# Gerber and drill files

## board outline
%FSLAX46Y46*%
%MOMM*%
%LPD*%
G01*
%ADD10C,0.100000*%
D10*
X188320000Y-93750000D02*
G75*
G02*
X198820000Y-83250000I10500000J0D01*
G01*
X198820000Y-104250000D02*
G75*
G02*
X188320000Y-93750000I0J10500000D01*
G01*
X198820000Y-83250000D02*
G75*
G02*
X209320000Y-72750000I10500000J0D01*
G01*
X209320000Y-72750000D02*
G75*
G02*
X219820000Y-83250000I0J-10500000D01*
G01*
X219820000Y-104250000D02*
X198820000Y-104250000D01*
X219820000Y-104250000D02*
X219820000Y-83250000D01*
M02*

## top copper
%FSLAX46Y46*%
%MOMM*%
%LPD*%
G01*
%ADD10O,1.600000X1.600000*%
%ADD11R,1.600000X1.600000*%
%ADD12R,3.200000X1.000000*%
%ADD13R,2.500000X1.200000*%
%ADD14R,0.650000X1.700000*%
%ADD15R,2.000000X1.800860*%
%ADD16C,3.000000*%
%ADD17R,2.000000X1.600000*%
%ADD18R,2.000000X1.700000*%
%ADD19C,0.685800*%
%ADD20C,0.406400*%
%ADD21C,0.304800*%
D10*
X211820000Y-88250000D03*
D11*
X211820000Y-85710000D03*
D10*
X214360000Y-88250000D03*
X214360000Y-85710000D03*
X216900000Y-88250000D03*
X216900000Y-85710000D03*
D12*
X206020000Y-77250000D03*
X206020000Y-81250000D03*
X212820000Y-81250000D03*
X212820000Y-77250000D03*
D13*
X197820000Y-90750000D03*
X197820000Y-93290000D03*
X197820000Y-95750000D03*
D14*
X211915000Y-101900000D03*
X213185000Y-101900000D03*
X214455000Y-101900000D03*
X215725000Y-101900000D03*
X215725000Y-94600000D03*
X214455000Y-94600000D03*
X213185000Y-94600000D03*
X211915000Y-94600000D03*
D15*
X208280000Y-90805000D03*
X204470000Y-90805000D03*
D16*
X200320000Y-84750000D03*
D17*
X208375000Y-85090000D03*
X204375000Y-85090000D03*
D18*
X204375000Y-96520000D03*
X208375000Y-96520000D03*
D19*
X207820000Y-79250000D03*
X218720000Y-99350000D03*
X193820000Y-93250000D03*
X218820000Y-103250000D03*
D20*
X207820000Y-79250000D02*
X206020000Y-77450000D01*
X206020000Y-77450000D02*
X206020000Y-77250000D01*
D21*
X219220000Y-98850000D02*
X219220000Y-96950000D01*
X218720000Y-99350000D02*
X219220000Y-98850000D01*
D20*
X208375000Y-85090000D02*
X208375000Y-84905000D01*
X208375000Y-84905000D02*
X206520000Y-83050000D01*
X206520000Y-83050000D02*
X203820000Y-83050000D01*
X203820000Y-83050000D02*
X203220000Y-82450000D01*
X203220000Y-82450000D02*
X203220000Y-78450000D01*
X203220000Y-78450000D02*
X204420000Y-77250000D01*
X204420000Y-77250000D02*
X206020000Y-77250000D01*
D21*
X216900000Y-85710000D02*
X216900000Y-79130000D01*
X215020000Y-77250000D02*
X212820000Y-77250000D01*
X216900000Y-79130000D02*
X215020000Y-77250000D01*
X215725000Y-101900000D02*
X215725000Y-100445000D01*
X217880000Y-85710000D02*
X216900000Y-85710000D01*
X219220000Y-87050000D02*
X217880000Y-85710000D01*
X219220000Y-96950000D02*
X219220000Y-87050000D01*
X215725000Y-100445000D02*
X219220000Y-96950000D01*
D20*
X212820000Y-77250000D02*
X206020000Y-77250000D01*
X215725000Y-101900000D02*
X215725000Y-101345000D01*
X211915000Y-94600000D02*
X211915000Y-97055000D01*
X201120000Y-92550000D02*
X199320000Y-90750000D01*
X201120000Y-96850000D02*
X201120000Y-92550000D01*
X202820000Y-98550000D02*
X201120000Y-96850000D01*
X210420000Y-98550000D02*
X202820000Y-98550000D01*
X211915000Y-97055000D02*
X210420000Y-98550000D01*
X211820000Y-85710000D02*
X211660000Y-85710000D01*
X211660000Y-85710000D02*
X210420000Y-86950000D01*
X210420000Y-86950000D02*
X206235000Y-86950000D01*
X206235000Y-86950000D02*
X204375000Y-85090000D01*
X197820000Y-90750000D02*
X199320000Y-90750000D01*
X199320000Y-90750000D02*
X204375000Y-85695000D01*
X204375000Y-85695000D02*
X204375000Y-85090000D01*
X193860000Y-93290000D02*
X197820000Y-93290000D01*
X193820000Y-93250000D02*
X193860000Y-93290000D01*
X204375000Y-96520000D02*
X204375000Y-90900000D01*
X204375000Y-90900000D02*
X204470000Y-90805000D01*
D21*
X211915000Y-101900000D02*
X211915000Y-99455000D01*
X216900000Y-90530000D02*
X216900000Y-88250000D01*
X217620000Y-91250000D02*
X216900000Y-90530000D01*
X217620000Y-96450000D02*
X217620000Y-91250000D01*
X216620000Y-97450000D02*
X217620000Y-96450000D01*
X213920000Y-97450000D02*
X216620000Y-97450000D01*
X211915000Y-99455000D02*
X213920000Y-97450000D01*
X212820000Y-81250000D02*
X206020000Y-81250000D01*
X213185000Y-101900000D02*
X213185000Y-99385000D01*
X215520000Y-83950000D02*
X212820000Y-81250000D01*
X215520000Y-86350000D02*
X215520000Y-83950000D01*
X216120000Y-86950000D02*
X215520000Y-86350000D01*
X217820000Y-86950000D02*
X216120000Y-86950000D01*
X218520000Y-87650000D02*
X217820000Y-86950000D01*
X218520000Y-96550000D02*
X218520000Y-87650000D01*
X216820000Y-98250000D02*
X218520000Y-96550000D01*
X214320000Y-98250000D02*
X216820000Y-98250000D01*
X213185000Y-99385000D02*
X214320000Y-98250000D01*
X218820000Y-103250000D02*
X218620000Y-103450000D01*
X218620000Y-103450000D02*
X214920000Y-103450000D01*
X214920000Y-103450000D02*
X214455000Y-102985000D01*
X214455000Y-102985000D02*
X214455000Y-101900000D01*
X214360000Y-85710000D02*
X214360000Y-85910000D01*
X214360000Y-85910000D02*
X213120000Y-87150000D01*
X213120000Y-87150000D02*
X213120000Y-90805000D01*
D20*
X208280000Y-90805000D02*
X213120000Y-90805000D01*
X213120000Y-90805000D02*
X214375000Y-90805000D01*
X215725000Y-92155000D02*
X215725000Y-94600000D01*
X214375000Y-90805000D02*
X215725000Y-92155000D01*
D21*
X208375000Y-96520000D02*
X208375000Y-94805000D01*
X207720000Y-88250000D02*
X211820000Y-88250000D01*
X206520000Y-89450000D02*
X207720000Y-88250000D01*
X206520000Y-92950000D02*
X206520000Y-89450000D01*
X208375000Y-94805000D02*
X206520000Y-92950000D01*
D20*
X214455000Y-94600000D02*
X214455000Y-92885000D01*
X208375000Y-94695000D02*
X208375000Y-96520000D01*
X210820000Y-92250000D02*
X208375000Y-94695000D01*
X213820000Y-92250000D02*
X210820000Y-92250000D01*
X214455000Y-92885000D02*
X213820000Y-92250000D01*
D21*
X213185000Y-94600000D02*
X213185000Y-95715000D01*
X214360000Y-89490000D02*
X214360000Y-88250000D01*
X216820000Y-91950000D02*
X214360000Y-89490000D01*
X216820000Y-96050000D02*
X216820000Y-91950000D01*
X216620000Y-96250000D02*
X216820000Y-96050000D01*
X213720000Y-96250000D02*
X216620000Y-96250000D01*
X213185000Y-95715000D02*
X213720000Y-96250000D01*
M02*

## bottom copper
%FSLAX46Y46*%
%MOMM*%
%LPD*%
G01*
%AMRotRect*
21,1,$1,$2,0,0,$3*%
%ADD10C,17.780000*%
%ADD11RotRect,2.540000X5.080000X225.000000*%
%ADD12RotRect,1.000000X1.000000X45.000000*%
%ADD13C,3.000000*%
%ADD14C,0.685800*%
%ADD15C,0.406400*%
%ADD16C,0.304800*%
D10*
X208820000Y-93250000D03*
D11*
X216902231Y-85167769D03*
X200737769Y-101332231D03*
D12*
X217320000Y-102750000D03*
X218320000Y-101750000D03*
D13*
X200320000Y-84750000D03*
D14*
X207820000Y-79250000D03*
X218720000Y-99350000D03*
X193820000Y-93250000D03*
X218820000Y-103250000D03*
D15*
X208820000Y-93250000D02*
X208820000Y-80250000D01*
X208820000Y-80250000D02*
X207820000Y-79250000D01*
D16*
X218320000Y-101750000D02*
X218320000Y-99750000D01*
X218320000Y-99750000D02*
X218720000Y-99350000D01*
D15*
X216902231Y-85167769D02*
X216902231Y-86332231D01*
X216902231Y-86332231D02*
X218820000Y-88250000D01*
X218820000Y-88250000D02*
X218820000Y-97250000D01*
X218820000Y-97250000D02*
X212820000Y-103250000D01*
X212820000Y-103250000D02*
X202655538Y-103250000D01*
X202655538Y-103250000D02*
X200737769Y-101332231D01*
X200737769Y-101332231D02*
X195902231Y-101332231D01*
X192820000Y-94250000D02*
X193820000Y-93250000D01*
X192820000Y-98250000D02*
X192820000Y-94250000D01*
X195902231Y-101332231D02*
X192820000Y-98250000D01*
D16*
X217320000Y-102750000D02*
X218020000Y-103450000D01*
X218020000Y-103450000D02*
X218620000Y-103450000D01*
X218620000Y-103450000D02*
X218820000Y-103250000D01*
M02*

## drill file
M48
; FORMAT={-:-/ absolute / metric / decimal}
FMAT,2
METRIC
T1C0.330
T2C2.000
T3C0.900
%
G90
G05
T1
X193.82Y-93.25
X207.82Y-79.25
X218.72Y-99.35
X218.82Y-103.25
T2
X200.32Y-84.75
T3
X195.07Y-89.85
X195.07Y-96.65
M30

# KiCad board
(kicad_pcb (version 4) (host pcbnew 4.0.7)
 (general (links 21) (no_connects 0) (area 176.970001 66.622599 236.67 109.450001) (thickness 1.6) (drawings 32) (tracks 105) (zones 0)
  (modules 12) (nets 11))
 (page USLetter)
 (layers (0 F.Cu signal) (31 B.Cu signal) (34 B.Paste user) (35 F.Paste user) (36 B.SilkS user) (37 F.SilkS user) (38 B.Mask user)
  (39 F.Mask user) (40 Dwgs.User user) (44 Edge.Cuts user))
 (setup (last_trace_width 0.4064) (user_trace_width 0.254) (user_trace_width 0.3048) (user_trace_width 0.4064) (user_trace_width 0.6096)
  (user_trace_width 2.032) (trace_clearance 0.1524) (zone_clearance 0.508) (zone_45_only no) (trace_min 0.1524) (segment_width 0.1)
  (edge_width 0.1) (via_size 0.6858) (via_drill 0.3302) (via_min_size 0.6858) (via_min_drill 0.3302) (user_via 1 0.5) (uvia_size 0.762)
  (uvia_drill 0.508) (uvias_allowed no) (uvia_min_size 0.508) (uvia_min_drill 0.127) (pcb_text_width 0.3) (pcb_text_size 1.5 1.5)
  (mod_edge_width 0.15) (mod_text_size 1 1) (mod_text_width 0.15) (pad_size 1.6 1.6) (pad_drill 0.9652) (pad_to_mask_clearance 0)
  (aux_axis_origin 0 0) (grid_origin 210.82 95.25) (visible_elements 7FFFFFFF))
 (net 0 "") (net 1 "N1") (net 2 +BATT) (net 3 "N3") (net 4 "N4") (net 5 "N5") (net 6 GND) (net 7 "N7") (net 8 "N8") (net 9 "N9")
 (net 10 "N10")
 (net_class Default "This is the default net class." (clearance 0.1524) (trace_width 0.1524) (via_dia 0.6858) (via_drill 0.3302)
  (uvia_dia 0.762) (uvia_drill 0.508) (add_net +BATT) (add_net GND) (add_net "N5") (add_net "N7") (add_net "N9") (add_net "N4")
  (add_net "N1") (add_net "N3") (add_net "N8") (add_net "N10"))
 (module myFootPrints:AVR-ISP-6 (layer F.Cu) (at 211.82 88.25 90)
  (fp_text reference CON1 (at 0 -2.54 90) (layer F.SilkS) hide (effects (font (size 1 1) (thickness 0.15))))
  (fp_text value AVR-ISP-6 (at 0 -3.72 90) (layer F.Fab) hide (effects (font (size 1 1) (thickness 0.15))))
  (pad 1 smd oval (at 0 0 90) (size 1.6 1.6) (layers F.Cu F.Paste F.Mask) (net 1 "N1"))
  (pad 2 smd rect (at 2.54 0 90) (size 1.6 1.6) (layers F.Cu F.Paste F.Mask) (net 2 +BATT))
  (pad 3 smd oval (at 0 2.54 90) (size 1.6 1.6) (layers F.Cu F.Paste F.Mask) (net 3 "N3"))
  (pad 4 smd oval (at 2.54 2.54 90) (size 1.6 1.6) (layers F.Cu F.Paste F.Mask) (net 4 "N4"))
  (pad 5 smd oval (at 0 5.08 90) (size 1.6 1.6) (layers F.Cu F.Paste F.Mask) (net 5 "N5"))
  (pad 6 smd oval (at 2.54 5.08 90) (size 1.6 1.6) (layers F.Cu F.Paste F.Mask) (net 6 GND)))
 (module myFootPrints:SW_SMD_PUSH (layer F.Cu) (at 212.82 81.25 180)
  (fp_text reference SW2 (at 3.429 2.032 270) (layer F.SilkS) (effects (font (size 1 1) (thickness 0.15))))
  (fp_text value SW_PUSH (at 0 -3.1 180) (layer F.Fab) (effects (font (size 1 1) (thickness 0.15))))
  (pad 2 smd rect (at 6.8 4 180) (size 3.2 1) (layers F.Cu F.Paste F.Mask) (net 6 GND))
  (pad 1 smd rect (at 6.8 0 180) (size 3.2 1) (layers F.Cu F.Paste F.Mask) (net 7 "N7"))
  (pad 1 smd rect (at 0 0 180) (size 3.2 1) (layers F.Cu F.Paste F.Mask) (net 7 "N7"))
  (pad 2 smd rect (at 0 4 180) (size 3.2 1) (layers F.Cu F.Paste F.Mask) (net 6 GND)))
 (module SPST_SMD (layer F.Cu) (at 197.82 93.25 270)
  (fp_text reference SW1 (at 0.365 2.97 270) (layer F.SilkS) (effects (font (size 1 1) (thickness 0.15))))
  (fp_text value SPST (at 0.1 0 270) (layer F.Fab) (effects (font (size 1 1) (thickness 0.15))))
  (pad "" np_thru_hole circle (at 3.4 2.75 270) (size 0.9 0.9) (drill 0.9) (layers *.Cu *.Mask))
  (pad 1 smd rect (at -2.5 0 270) (size 1.2 2.5) (layers F.Cu F.Paste F.Mask) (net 2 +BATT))
  (pad 2 smd rect (at 0.04 0 270) (size 1.2 2.5) (layers F.Cu F.Paste F.Mask) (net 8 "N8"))
  (pad 3 smd rect (at 2.5 0 270) (size 1.2 2.5) (layers F.Cu F.Paste F.Mask))
  (pad "" np_thru_hole circle (at -3.4 2.75 270) (size 0.9 0.9) (drill 0.9) (layers *.Cu *.Mask)))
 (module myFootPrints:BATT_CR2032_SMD (layer B.Cu) (at 208.82 93.25 225)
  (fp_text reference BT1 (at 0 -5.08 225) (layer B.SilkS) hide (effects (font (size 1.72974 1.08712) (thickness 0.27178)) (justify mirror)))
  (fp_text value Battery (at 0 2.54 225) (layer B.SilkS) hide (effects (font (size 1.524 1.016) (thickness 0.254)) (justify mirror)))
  (pad 2 smd circle (at 0 0 225) (size 17.78 17.78) (layers B.Cu B.Paste B.Mask) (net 6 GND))
  (pad 1 smd rect (at -11.43 0 225) (size 2.54 5.08) (layers B.Cu B.Paste B.Mask) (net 8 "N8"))
  (pad 1 smd rect (at 11.43 0 225) (size 2.54 5.08) (layers B.Cu B.Paste B.Mask) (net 8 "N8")))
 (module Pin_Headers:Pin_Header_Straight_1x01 (layer F.Cu) (at 217.32 102.75 45)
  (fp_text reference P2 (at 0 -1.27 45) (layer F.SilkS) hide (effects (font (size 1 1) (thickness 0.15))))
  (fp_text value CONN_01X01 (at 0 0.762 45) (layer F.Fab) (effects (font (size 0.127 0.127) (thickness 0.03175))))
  (pad 1 smd rect (at 0 0 45) (size 1 1) (layers B.Cu B.Paste B.Mask) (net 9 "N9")))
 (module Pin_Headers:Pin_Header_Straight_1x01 (layer F.Cu) (at 218.32 101.75 45)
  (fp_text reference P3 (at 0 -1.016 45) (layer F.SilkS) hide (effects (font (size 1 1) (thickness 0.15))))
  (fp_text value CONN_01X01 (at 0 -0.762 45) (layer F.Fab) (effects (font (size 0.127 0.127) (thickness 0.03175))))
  (pad 1 smd rect (at 0 0 45) (size 1 1) (layers B.Cu B.Paste B.Mask) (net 6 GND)))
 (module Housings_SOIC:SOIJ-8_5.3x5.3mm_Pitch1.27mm (layer F.Cu) (at 213.82 98.25 90)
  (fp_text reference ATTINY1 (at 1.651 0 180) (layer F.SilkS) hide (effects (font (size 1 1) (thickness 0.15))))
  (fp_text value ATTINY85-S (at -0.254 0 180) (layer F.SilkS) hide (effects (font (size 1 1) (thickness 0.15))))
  (pad 1 smd rect (at -3.65 -1.905 90) (size 1.7 0.65) (layers F.Cu F.Paste F.Mask) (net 5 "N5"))
  (pad 2 smd rect (at -3.65 -0.635 90) (size 1.7 0.65) (layers F.Cu F.Paste F.Mask) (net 7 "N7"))
  (pad 3 smd rect (at -3.65 0.635 90) (size 1.7 0.65) (layers F.Cu F.Paste F.Mask) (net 9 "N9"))
  (pad 4 smd rect (at -3.65 1.905 90) (size 1.7 0.65) (layers F.Cu F.Paste F.Mask) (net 6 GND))
  (pad 5 smd rect (at 3.65 1.905 90) (size 1.7 0.65) (layers F.Cu F.Paste F.Mask) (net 4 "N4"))
  (pad 6 smd rect (at 3.65 0.635 90) (size 1.7 0.65) (layers F.Cu F.Paste F.Mask) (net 1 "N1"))
  (pad 7 smd rect (at 3.65 -0.635 90) (size 1.7 0.65) (layers F.Cu F.Paste F.Mask) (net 3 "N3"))
  (pad 8 smd rect (at 3.65 -1.905 90) (size 1.7 0.65) (layers F.Cu F.Paste F.Mask) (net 2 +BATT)))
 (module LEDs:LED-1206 (layer F.Cu) (at 206.375 90.805)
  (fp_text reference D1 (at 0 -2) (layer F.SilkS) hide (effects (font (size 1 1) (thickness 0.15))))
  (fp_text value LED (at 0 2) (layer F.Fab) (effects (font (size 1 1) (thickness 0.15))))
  (pad 2 smd rect (at 1.905 0 180) (size 2 1.80086) (layers F.Cu F.Paste F.Mask) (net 4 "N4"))
  (pad 1 smd rect (at -1.905 0 180) (size 2 1.80086) (layers F.Cu F.Paste F.Mask) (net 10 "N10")))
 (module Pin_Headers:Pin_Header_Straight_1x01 (layer F.Cu) (at 200.32 84.75)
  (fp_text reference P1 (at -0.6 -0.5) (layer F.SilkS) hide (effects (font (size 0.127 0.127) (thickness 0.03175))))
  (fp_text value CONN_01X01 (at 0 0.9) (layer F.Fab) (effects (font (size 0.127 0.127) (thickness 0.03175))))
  (pad "" thru_hole circle (at 0 0) (size 3 3) (drill 2) (layers *.Cu *.Mask)))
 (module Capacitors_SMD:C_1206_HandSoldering (layer F.Cu) (at 206.375 85.09 180)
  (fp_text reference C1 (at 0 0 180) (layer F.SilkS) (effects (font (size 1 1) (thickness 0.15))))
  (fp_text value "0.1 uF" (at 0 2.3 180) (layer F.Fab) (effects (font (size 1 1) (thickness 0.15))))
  (pad 1 smd rect (at -2 0 180) (size 2 1.6) (layers F.Cu F.Paste F.Mask) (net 6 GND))
  (pad 2 smd rect (at 2 0 180) (size 2 1.6) (layers F.Cu F.Paste F.Mask) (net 2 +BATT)))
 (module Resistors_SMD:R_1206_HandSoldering (layer F.Cu) (at 206.375 96.52)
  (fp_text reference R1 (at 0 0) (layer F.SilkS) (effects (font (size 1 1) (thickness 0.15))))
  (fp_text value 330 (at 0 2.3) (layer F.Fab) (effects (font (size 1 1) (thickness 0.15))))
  (pad 1 smd rect (at -2 0) (size 2 1.7) (layers F.Cu F.Paste F.Mask) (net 10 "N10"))
  (pad 2 smd rect (at 2 0) (size 2 1.7) (layers F.Cu F.Paste F.Mask) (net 1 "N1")))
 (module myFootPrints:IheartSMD (layer F.Cu) (at 202.82 101.25)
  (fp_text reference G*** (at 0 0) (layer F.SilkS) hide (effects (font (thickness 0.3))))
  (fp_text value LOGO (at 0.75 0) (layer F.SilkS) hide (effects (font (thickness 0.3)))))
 (gr_arc (start 198.82 93.75) (end 188.32 93.75) (angle 90) (layer Edge.Cuts) (width 0.1))
 (gr_arc (start 198.82 93.75) (end 198.82 104.25) (angle 90) (layer Edge.Cuts) (width 0.1))
 (gr_arc (start 209.32 83.25) (end 198.82 83.25) (angle 90) (layer Edge.Cuts) (width 0.1))
 (gr_arc (start 209.32 83.25) (end 209.32 72.75) (angle 90) (layer Edge.Cuts) (width 0.1))
 (gr_line (start 219.82 104.25) (end 198.82 104.25) (angle 90) (layer Edge.Cuts) (width 0.1))
 (gr_line (start 219.82 104.25) (end 219.82 83.25) (angle 90) (layer Edge.Cuts) (width 0.1))
 (segment (start 208.82 93.25) (end 208.82 80.25) (width 0.4064) (layer B.Cu) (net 6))
 (segment (start 207.82 79.25) (end 206.02 77.45) (width 0.4064) (layer F.Cu) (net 6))
 (via (at 207.82 79.25) (size 0.6858) (drill 0.3302) (layers F.Cu B.Cu) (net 6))
 (segment (start 208.82 80.25) (end 207.82 79.25) (width 0.4064) (layer B.Cu) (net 6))
 (segment (start 206.02 77.45) (end 206.02 77.25) (width 0.4064) (layer F.Cu) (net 6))
 (segment (start 218.32 101.75) (end 218.32 99.75) (width 0.3048) (layer B.Cu) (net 6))
 (segment (start 219.22 98.85) (end 219.22 96.95) (width 0.3048) (layer F.Cu) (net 6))
 (segment (start 218.72 99.35) (end 219.22 98.85) (width 0.3048) (layer F.Cu) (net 6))
 (via (at 218.72 99.35) (size 0.6858) (drill 0.3302) (layers F.Cu B.Cu) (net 6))
 (segment (start 218.32 99.75) (end 218.72 99.35) (width 0.3048) (layer B.Cu) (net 6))
 (segment (start 208.375 85.09) (end 208.375 84.905) (width 0.4064) (layer F.Cu) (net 6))
 (segment (start 208.375 84.905) (end 206.52 83.05) (width 0.4064) (layer F.Cu) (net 6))
 (segment (start 206.52 83.05) (end 203.82 83.05) (width 0.4064) (layer F.Cu) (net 6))
 (segment (start 203.82 83.05) (end 203.22 82.45) (width 0.4064) (layer F.Cu) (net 6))
 (segment (start 203.22 82.45) (end 203.22 78.45) (width 0.4064) (layer F.Cu) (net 6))
 (segment (start 203.22 78.45) (end 204.42 77.25) (width 0.4064) (layer F.Cu) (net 6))
 (segment (start 204.42 77.25) (end 206.02 77.25) (width 0.4064) (layer F.Cu) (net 6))
 (segment (start 216.9 85.71) (end 216.9 79.13) (width 0.3048) (layer F.Cu) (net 6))
 (segment (start 215.02 77.25) (end 212.82 77.25) (width 0.3048) (layer F.Cu) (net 6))
 (segment (start 216.9 79.13) (end 215.02 77.25) (width 0.3048) (layer F.Cu) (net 6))
 (segment (start 215.725 101.9) (end 215.725 100.445) (width 0.3048) (layer F.Cu) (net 6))
 (segment (start 217.88 85.71) (end 216.9 85.71) (width 0.3048) (layer F.Cu) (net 6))
 (segment (start 219.22 87.05) (end 217.88 85.71) (width 0.3048) (layer F.Cu) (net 6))
 (segment (start 219.22 96.95) (end 219.22 87.05) (width 0.3048) (layer F.Cu) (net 6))
 (segment (start 215.725 100.445) (end 219.22 96.95) (width 0.3048) (layer F.Cu) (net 6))
 (segment (start 212.82 77.25) (end 206.02 77.25) (width 0.4064) (layer F.Cu) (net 6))
 (segment (start 215.725 101.9) (end 215.725 101.345) (width 0.4064) (layer F.Cu) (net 6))
 (segment (start 211.915 94.6) (end 211.915 97.055) (width 0.4064) (layer F.Cu) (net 2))
 (segment (start 201.12 92.55) (end 199.32 90.75) (width 0.4064) (layer F.Cu) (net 2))
 (segment (start 201.12 96.85) (end 201.12 92.55) (width 0.4064) (layer F.Cu) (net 2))
 (segment (start 202.82 98.55) (end 201.12 96.85) (width 0.4064) (layer F.Cu) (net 2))
 (segment (start 210.42 98.55) (end 202.82 98.55) (width 0.4064) (layer F.Cu) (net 2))
 (segment (start 211.915 97.055) (end 210.42 98.55) (width 0.4064) (layer F.Cu) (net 2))
 (segment (start 211.82 85.71) (end 211.66 85.71) (width 0.4064) (layer F.Cu) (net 2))
 (segment (start 211.66 85.71) (end 210.42 86.95) (width 0.4064) (layer F.Cu) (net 2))
 (segment (start 210.42 86.95) (end 206.235 86.95) (width 0.4064) (layer F.Cu) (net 2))
 (segment (start 206.235 86.95) (end 204.375 85.09) (width 0.4064) (layer F.Cu) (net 2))
 (segment (start 197.82 90.75) (end 199.32 90.75) (width 0.4064) (layer F.Cu) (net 2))
 (segment (start 199.32 90.75) (end 204.375 85.695) (width 0.4064) (layer F.Cu) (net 2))
 (segment (start 204.375 85.695) (end 204.375 85.09) (width 0.4064) (layer F.Cu) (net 2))
 (segment (start 216.902231 85.167769) (end 216.902231 86.332231) (width 0.4064) (layer B.Cu) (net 8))
 (segment (start 216.902231 86.332231) (end 218.82 88.25) (width 0.4064) (layer B.Cu) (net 8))
 (segment (start 218.82 88.25) (end 218.82 97.25) (width 0.4064) (layer B.Cu) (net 8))
 (segment (start 218.82 97.25) (end 212.82 103.25) (width 0.4064) (layer B.Cu) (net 8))
 (segment (start 212.82 103.25) (end 202.655538 103.25) (width 0.4064) (layer B.Cu) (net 8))
 (segment (start 202.655538 103.25) (end 200.737769 101.332231) (width 0.4064) (layer B.Cu) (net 8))
 (segment (start 200.737769 101.332231) (end 195.902231 101.332231) (width 0.4064) (layer B.Cu) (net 8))
 (segment (start 193.86 93.29) (end 197.82 93.29) (width 0.4064) (layer F.Cu) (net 8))
 (segment (start 193.82 93.25) (end 193.86 93.29) (width 0.4064) (layer F.Cu) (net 8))
 (via (at 193.82 93.25) (size 0.6858) (drill 0.3302) (layers F.Cu B.Cu) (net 8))
 (segment (start 192.82 94.25) (end 193.82 93.25) (width 0.4064) (layer B.Cu) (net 8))
 (segment (start 192.82 98.25) (end 192.82 94.25) (width 0.4064) (layer B.Cu) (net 8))
 (segment (start 195.902231 101.332231) (end 192.82 98.25) (width 0.4064) (layer B.Cu) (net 8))
 (segment (start 204.375 96.52) (end 204.375 90.9) (width 0.4064) (layer F.Cu) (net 10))
 (segment (start 204.375 90.9) (end 204.47 90.805) (width 0.4064) (layer F.Cu) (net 10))
 (segment (start 211.915 101.9) (end 211.915 99.455) (width 0.3048) (layer F.Cu) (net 5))
 (segment (start 216.9 90.53) (end 216.9 88.25) (width 0.3048) (layer F.Cu) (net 5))
 (segment (start 217.62 91.25) (end 216.9 90.53) (width 0.3048) (layer F.Cu) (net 5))
 (segment (start 217.62 96.45) (end 217.62 91.25) (width 0.3048) (layer F.Cu) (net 5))
 (segment (start 216.62 97.45) (end 217.62 96.45) (width 0.3048) (layer F.Cu) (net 5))
 (segment (start 213.92 97.45) (end 216.62 97.45) (width 0.3048) (layer F.Cu) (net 5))
 (segment (start 211.915 99.455) (end 213.92 97.45) (width 0.3048) (layer F.Cu) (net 5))
 (segment (start 212.82 81.25) (end 206.02 81.25) (width 0.3048) (layer F.Cu) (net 7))
 (segment (start 213.185 101.9) (end 213.185 99.385) (width 0.3048) (layer F.Cu) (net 7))
 (segment (start 215.52 83.95) (end 212.82 81.25) (width 0.3048) (layer F.Cu) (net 7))
 (segment (start 215.52 86.35) (end 215.52 83.95) (width 0.3048) (layer F.Cu) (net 7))
 (segment (start 216.12 86.95) (end 215.52 86.35) (width 0.3048) (layer F.Cu) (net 7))
 (segment (start 217.82 86.95) (end 216.12 86.95) (width 0.3048) (layer F.Cu) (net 7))
 (segment (start 218.52 87.65) (end 217.82 86.95) (width 0.3048) (layer F.Cu) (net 7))
 (segment (start 218.52 96.55) (end 218.52 87.65) (width 0.3048) (layer F.Cu) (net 7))
 (segment (start 216.82 98.25) (end 218.52 96.55) (width 0.3048) (layer F.Cu) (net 7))
 (segment (start 214.32 98.25) (end 216.82 98.25) (width 0.3048) (layer F.Cu) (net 7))
 (segment (start 213.185 99.385) (end 214.32 98.25) (width 0.3048) (layer F.Cu) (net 7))
 (segment (start 217.32 102.75) (end 218.02 103.45) (width 0.3048) (layer B.Cu) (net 9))
 (segment (start 218.02 103.45) (end 218.62 103.45) (width 0.3048) (layer B.Cu) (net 9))
 (segment (start 218.62 103.45) (end 218.82 103.25) (width 0.3048) (layer B.Cu) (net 9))
 (via (at 218.82 103.25) (size 0.6858) (drill 0.3302) (layers F.Cu B.Cu) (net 9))
 (segment (start 218.82 103.25) (end 218.62 103.45) (width 0.3048) (layer F.Cu) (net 9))
 (segment (start 218.62 103.45) (end 214.92 103.45) (width 0.3048) (layer F.Cu) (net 9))
 (segment (start 214.92 103.45) (end 214.455 102.985) (width 0.3048) (layer F.Cu) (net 9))
 (segment (start 214.455 102.985) (end 214.455 101.9) (width 0.3048) (layer F.Cu) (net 9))
 (segment (start 214.36 85.71) (end 214.36 85.91) (width 0.3048) (layer F.Cu) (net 4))
 (segment (start 214.36 85.91) (end 213.12 87.15) (width 0.3048) (layer F.Cu) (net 4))
 (segment (start 213.12 87.15) (end 213.12 90.805) (width 0.3048) (layer F.Cu) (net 4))
 (segment (start 208.28 90.805) (end 213.12 90.805) (width 0.4064) (layer F.Cu) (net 4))
 (segment (start 213.12 90.805) (end 214.375 90.805) (width 0.4064) (layer F.Cu) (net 4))
 (segment (start 215.725 92.155) (end 215.725 94.6) (width 0.4064) (layer F.Cu) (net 4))
 (segment (start 214.375 90.805) (end 215.725 92.155) (width 0.4064) (layer F.Cu) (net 4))
 (segment (start 208.375 96.52) (end 208.375 94.805) (width 0.3048) (layer F.Cu) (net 1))
 (segment (start 207.72 88.25) (end 211.82 88.25) (width 0.3048) (layer F.Cu) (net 1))
 (segment (start 206.52 89.45) (end 207.72 88.25) (width 0.3048) (layer F.Cu) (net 1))
 (segment (start 206.52 92.95) (end 206.52 89.45) (width 0.3048) (layer F.Cu) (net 1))
 (segment (start 208.375 94.805) (end 206.52 92.95) (width 0.3048) (layer F.Cu) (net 1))
 (segment (start 214.455 94.6) (end 214.455 92.885) (width 0.4064) (layer F.Cu) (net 1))
 (segment (start 208.375 94.695) (end 208.375 96.52) (width 0.4064) (layer F.Cu) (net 1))
 (segment (start 210.82 92.25) (end 208.375 94.695) (width 0.4064) (layer F.Cu) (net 1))
 (segment (start 213.82 92.25) (end 210.82 92.25) (width 0.4064) (layer F.Cu) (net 1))
 (segment (start 214.455 92.885) (end 213.82 92.25) (width 0.4064) (layer F.Cu) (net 1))
 (segment (start 213.185 94.6) (end 213.185 95.715) (width 0.3048) (layer F.Cu) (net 3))
 (segment (start 214.36 89.49) (end 214.36 88.25) (width 0.3048) (layer F.Cu) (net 3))
 (segment (start 216.82 91.95) (end 214.36 89.49) (width 0.3048) (layer F.Cu) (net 3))
 (segment (start 216.82 96.05) (end 216.82 91.95) (width 0.3048) (layer F.Cu) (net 3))
 (segment (start 216.62 96.25) (end 216.82 96.05) (width 0.3048) (layer F.Cu) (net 3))
 (segment (start 213.72 96.25) (end 216.62 96.25) (width 0.3048) (layer F.Cu) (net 3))
 (segment (start 213.185 95.715) (end 213.72 96.25) (width 0.3048) (layer F.Cu) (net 3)))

